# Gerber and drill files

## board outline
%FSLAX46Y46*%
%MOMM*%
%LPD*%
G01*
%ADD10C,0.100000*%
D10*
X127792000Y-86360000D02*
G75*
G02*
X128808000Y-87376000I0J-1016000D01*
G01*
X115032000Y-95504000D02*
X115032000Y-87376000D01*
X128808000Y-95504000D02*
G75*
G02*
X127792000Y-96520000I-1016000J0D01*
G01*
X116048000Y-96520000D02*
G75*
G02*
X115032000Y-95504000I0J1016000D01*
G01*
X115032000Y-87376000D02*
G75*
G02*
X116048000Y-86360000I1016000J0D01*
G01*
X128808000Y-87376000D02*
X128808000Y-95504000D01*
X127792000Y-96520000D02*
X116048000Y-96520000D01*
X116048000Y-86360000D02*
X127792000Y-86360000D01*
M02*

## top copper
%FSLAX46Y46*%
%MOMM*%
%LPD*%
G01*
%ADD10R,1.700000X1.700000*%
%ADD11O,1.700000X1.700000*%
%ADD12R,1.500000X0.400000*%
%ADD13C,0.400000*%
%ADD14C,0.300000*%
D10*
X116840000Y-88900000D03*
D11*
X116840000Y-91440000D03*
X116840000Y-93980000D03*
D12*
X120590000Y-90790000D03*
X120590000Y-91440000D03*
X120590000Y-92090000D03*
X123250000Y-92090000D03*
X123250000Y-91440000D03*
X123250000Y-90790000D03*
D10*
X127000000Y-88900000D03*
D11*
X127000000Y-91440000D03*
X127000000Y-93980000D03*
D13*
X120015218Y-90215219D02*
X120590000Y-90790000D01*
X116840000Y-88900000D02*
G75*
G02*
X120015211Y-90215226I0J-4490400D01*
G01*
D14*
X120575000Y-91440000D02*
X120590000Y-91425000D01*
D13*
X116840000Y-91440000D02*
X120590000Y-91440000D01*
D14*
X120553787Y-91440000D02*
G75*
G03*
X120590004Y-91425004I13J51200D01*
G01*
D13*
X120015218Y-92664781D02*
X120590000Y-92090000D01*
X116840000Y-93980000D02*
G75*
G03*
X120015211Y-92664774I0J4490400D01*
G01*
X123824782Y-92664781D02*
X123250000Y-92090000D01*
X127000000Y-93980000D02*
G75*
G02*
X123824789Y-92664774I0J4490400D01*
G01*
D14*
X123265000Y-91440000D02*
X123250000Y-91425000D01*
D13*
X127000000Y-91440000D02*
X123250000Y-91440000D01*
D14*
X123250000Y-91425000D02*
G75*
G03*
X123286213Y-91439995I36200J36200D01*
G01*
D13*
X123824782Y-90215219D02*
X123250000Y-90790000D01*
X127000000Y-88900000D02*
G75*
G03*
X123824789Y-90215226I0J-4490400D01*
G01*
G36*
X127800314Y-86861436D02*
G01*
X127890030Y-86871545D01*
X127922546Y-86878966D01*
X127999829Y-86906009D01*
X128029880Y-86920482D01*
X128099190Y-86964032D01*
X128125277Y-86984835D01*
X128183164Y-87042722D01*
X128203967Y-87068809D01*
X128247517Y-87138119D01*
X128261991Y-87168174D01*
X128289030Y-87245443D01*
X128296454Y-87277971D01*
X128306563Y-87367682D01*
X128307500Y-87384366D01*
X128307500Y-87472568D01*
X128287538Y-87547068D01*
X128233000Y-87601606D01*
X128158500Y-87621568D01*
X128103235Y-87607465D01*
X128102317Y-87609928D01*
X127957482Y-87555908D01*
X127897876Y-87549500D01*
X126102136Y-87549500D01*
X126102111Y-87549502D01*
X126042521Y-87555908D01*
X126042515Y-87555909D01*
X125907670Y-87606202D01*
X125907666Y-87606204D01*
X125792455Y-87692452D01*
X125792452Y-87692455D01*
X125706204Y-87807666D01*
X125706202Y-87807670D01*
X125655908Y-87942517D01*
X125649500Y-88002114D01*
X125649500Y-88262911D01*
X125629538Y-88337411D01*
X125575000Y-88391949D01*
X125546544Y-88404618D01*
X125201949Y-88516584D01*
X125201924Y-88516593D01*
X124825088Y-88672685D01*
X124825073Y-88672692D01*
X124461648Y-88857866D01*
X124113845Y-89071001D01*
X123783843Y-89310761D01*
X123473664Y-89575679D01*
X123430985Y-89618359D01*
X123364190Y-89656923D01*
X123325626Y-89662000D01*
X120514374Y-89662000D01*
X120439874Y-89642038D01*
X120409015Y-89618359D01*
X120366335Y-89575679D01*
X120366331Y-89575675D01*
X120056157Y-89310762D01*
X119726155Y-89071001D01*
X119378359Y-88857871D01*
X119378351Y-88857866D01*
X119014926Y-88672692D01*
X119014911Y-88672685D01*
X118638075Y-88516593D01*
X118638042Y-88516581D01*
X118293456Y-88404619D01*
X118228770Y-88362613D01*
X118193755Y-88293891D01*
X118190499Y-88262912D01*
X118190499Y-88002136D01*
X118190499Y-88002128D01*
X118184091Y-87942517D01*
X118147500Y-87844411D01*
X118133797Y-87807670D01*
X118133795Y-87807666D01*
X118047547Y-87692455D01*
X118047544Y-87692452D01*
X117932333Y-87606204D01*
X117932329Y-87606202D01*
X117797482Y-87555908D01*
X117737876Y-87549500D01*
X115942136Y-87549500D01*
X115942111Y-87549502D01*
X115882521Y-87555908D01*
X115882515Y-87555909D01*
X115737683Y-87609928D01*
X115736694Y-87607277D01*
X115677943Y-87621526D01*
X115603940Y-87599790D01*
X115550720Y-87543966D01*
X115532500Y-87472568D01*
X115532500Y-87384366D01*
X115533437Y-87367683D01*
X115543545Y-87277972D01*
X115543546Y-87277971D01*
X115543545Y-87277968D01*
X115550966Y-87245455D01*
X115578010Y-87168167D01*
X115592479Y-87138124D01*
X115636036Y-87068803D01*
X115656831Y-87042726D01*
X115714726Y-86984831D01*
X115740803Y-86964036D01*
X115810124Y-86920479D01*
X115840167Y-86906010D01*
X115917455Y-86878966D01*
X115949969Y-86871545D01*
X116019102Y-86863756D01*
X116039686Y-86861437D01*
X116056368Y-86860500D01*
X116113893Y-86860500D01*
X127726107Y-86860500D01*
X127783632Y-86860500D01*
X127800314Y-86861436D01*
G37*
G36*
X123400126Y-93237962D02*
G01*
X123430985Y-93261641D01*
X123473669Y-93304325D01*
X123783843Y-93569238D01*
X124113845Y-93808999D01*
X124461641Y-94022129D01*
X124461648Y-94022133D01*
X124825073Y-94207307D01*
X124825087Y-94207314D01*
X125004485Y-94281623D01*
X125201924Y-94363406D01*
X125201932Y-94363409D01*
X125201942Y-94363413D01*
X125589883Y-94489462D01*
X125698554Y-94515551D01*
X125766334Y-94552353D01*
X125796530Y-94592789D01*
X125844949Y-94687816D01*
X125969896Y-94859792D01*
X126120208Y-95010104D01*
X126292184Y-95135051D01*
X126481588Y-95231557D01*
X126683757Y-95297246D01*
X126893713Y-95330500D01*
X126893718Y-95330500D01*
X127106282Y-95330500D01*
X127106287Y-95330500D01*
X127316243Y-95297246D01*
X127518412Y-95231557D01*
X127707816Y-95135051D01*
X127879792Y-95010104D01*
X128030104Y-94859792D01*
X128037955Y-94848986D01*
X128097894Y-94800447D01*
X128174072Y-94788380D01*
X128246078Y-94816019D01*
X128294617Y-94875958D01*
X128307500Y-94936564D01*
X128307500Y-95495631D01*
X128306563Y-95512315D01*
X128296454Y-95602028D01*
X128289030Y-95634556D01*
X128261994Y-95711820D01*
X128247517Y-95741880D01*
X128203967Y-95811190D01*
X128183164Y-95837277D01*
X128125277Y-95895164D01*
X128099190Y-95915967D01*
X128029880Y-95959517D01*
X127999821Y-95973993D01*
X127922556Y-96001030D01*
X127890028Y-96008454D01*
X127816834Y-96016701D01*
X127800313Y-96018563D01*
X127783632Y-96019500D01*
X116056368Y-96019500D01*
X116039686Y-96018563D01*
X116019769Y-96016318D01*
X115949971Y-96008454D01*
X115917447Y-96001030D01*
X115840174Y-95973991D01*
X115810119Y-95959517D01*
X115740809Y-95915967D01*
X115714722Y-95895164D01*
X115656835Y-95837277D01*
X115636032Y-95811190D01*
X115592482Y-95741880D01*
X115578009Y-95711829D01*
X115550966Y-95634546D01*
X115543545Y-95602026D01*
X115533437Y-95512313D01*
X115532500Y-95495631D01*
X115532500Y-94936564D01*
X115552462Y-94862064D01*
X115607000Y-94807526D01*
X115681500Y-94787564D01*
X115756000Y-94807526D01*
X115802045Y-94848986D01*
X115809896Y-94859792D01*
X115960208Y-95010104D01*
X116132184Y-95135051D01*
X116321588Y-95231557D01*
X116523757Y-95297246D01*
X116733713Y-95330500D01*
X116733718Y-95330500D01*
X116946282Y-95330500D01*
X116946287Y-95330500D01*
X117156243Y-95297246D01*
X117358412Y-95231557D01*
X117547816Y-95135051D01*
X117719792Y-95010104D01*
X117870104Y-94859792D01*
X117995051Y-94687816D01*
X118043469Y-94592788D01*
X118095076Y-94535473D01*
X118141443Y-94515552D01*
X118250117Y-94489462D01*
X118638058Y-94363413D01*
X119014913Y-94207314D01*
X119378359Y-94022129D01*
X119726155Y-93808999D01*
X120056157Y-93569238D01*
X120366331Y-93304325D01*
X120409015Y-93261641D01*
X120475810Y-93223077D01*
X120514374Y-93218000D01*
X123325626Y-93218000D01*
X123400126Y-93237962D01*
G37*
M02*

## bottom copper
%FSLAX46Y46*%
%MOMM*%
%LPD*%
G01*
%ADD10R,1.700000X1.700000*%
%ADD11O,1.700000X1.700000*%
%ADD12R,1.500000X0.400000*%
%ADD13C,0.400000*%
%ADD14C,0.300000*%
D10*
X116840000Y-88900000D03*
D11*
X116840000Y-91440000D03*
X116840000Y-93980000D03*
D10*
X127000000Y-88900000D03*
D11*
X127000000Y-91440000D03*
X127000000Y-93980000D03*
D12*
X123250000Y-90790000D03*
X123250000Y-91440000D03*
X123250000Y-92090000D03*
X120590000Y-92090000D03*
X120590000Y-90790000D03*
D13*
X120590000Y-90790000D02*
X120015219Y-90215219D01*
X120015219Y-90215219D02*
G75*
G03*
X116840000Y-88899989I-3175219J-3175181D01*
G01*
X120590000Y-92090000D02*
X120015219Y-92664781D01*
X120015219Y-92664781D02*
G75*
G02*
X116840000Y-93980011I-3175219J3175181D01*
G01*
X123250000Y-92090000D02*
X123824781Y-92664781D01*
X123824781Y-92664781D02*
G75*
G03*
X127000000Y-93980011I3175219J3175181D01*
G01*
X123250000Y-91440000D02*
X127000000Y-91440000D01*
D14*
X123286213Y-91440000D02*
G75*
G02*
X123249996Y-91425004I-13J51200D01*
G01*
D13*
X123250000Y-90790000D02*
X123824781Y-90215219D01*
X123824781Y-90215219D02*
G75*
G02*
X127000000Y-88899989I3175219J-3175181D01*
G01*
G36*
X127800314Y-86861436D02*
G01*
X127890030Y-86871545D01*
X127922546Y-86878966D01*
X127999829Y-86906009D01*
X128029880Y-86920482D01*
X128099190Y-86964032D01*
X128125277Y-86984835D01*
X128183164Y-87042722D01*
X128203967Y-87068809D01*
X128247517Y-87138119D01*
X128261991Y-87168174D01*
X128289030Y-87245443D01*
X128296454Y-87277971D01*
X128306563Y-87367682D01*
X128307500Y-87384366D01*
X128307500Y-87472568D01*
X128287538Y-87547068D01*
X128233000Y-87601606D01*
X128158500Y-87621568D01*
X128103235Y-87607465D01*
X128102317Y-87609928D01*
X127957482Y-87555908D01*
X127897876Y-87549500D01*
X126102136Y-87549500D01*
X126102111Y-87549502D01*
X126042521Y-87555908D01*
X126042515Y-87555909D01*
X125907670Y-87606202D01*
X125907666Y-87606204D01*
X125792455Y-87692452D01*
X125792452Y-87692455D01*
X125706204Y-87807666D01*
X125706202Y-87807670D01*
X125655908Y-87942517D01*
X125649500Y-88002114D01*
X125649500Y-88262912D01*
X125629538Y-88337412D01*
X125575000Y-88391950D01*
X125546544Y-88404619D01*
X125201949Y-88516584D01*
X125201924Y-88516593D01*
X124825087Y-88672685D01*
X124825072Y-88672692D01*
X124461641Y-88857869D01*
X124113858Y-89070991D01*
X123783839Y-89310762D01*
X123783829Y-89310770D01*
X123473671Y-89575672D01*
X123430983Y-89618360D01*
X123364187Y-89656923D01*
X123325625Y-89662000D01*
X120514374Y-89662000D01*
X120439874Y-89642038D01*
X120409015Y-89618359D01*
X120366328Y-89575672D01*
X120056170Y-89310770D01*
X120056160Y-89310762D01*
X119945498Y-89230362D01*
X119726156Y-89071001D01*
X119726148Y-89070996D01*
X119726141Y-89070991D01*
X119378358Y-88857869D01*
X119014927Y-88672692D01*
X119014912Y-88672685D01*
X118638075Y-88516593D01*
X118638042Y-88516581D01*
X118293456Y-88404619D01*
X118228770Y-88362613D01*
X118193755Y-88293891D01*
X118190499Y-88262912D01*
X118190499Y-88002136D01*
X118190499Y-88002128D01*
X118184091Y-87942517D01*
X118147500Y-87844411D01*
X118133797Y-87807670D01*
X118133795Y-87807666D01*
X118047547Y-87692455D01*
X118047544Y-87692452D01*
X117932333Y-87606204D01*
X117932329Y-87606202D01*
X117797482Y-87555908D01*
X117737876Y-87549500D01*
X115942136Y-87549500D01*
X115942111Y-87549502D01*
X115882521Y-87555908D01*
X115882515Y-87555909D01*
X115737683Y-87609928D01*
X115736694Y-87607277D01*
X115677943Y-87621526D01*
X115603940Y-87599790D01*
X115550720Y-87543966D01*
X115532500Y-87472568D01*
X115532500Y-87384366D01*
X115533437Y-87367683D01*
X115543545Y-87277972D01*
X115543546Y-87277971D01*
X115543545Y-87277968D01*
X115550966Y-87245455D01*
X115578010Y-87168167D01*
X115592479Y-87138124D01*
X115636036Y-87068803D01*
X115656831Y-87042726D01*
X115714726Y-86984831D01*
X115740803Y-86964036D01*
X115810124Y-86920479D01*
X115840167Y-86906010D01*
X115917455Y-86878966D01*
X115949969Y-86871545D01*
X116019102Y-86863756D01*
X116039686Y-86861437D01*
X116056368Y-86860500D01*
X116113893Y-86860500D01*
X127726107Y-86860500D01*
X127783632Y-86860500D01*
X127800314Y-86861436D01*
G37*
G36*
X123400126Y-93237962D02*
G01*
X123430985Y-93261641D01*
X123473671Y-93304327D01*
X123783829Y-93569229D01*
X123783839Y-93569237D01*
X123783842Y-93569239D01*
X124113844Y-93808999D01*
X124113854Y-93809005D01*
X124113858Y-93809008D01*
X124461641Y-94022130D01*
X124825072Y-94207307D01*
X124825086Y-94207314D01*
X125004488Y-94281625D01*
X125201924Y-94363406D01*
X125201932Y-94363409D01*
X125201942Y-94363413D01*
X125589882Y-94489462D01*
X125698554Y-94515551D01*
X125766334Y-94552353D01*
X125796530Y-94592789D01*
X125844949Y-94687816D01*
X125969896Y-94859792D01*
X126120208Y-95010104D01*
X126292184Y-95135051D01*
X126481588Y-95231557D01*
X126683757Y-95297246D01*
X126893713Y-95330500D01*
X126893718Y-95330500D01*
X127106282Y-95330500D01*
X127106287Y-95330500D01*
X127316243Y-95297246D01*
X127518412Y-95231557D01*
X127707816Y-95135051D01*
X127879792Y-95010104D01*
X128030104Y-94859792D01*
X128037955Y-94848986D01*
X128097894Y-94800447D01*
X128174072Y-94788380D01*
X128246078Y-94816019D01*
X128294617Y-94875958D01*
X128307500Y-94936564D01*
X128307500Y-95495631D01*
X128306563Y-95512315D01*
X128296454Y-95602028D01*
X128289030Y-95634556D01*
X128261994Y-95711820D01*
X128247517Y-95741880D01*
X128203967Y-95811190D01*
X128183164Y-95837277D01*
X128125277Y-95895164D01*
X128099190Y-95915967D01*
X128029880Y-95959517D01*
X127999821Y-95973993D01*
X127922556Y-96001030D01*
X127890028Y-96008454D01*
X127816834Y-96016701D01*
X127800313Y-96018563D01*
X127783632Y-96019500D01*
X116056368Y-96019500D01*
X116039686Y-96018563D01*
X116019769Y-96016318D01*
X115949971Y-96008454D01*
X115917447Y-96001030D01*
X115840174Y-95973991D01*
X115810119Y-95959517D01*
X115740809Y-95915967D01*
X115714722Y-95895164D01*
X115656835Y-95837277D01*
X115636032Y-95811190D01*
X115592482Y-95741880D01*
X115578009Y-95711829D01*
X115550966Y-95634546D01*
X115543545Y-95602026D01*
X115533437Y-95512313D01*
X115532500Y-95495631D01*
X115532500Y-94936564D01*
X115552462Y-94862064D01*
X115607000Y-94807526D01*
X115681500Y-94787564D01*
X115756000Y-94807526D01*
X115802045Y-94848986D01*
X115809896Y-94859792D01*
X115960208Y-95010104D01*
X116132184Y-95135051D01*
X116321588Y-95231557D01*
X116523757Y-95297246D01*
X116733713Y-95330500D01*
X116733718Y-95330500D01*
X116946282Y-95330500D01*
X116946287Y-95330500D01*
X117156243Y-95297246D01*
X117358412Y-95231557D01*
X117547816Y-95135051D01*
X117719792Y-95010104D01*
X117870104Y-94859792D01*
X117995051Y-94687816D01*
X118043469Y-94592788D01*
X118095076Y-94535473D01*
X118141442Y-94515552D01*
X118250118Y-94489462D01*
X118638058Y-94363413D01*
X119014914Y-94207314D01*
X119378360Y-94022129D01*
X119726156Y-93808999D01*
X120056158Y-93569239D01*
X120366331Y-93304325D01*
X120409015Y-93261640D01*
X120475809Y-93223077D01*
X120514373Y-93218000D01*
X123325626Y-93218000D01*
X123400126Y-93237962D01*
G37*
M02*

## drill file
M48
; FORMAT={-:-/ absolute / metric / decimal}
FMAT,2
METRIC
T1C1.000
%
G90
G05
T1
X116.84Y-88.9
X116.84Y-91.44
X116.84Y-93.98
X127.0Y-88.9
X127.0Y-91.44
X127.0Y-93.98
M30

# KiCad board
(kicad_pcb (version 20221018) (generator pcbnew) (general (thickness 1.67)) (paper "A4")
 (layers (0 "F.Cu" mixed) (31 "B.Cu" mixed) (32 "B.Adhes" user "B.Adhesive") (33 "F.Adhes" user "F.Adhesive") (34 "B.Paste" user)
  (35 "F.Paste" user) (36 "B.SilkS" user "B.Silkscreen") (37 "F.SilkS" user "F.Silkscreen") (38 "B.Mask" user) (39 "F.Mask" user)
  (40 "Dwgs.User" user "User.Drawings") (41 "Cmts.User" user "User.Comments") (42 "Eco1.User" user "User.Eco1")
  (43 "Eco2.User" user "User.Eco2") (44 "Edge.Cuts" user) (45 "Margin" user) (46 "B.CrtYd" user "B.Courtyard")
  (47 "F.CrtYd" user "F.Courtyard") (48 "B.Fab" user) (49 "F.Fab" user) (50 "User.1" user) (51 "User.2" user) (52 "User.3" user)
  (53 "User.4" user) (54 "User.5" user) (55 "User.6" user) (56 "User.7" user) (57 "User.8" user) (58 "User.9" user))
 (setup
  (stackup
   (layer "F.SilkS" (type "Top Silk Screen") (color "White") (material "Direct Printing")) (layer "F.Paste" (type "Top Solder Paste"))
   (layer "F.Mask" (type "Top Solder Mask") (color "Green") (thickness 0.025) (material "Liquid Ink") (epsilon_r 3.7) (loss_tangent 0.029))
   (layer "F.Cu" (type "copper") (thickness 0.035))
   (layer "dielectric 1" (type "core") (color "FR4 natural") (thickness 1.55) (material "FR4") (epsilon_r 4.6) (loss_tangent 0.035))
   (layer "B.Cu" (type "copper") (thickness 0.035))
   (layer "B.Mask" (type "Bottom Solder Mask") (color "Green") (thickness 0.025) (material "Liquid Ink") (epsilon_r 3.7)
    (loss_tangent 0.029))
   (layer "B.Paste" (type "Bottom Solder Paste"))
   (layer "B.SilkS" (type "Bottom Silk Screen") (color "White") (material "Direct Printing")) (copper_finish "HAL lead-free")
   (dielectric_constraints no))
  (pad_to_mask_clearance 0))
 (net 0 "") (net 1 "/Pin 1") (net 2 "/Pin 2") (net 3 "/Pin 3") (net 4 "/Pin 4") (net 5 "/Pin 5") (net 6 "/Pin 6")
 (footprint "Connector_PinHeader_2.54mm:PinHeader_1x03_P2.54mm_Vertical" (layer "F.Cu") (at 116.84 88.9)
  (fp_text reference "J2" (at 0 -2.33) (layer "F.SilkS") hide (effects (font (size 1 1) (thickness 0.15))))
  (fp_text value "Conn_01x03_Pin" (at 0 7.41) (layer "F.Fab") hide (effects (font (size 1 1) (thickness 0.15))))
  (pad "1" thru_hole rect (at 0 0) (size 1.7 1.7) (drill 1) (layers "*.Cu" "*.Mask") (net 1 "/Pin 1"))
  (pad "2" thru_hole oval (at 0 2.54) (size 1.7 1.7) (drill 1) (layers "*.Cu" "*.Mask") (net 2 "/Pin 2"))
  (pad "3" thru_hole oval (at 0 5.08) (size 1.7 1.7) (drill 1) (layers "*.Cu" "*.Mask") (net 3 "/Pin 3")))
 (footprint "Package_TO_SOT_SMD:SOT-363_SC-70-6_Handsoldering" (layer "F.Cu") (at 121.92 91.44)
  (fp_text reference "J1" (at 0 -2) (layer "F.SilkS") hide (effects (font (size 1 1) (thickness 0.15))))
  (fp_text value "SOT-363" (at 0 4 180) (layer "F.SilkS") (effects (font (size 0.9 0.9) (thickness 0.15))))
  (pad "1" smd rect (at -1.33 -0.65) (size 1.5 0.4) (layers "F.Cu" "F.Paste" "F.Mask") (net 1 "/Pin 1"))
  (pad "2" smd rect (at -1.33 0) (size 1.5 0.4) (layers "F.Cu" "F.Paste" "F.Mask") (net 2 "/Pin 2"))
  (pad "3" smd rect (at -1.33 0.65) (size 1.5 0.4) (layers "F.Cu" "F.Paste" "F.Mask") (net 3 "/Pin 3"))
  (pad "4" smd rect (at 1.33 0.65) (size 1.5 0.4) (layers "F.Cu" "F.Paste" "F.Mask") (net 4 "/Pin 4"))
  (pad "5" smd rect (at 1.33 0) (size 1.5 0.4) (layers "F.Cu" "F.Paste" "F.Mask") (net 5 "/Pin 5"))
  (pad "6" smd rect (at 1.33 -0.65) (size 1.5 0.4) (layers "F.Cu" "F.Paste" "F.Mask") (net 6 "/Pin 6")))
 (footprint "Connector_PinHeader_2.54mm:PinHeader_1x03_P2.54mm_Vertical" (layer "F.Cu") (at 127 88.9)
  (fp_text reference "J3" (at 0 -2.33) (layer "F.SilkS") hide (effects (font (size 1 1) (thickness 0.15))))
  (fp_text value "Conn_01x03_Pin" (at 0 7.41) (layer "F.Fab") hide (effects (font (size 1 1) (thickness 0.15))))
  (pad "1" thru_hole rect (at 0 0) (size 1.7 1.7) (drill 1) (layers "*.Cu" "*.Mask") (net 6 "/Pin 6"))
  (pad "2" thru_hole oval (at 0 2.54) (size 1.7 1.7) (drill 1) (layers "*.Cu" "*.Mask") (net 5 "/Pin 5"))
  (pad "3" thru_hole oval (at 0 5.08) (size 1.7 1.7) (drill 1) (layers "*.Cu" "*.Mask") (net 4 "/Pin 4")))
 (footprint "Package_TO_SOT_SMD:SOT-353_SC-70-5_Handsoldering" (layer "B.Cu") (at 121.92 91.44 180)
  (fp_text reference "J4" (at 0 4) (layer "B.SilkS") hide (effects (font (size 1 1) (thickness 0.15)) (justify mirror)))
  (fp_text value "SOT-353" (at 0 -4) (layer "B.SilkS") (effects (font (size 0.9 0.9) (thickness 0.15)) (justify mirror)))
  (pad "1" smd rect (at -1.33 0.65 180) (size 1.5 0.4) (layers "B.Cu" "B.Paste" "B.Mask") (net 6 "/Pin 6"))
  (pad "2" smd rect (at -1.33 0 180) (size 1.5 0.4) (layers "B.Cu" "B.Paste" "B.Mask") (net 5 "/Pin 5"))
  (pad "3" smd rect (at -1.33 -0.65 180) (size 1.5 0.4) (layers "B.Cu" "B.Paste" "B.Mask") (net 4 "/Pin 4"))
  (pad "4" smd rect (at 1.33 -0.65 180) (size 1.5 0.4) (layers "B.Cu" "B.Paste" "B.Mask") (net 3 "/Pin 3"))
  (pad "5" smd rect (at 1.33 0.65 180) (size 1.5 0.4) (layers "B.Cu" "B.Paste" "B.Mask") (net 1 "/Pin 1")))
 (gr_arc (start 127.792 86.36) (mid 128.51042 86.65758) (end 128.808 87.376) (stroke (width 0.1) (type default)) (layer "Edge.Cuts"))
 (gr_line (start 115.032 95.504) (end 115.032 87.376) (stroke (width 0.1) (type default)) (layer "Edge.Cuts"))
 (gr_arc (start 128.808 95.504) (mid 128.51042 96.22242) (end 127.792 96.52) (stroke (width 0.1) (type default)) (layer "Edge.Cuts"))
 (gr_arc (start 116.048 96.52) (mid 115.32958 96.22242) (end 115.032 95.504) (stroke (width 0.1) (type default)) (layer "Edge.Cuts"))
 (gr_arc (start 115.032 87.376) (mid 115.32958 86.65758) (end 116.048 86.36) (stroke (width 0.1) (type default)) (layer "Edge.Cuts"))
 (gr_line (start 128.808 87.376) (end 128.808 95.504) (stroke (width 0.1) (type default)) (layer "Edge.Cuts"))
 (gr_line (start 127.792 96.52) (end 116.048 96.52) (stroke (width 0.1) (type default)) (layer "Edge.Cuts"))
 (gr_line (start 116.048 86.36) (end 127.792 86.36) (stroke (width 0.1) (type default)) (layer "Edge.Cuts"))
 (segment (start 120.015218 90.215219) (end 120.59 90.79) (width 0.4) (layer "F.Cu") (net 1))
 (arc (start 116.84 88.9) (mid 118.558416 89.241814) (end 120.015218 90.215219) (width 0.4) (layer "F.Cu") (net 1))
 (segment (start 120.59 90.79) (end 120.015219 90.215219) (width 0.4) (layer "B.Cu") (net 1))
 (arc (start 120.015219 90.215219) (mid 118.558416 89.241814) (end 116.84 88.9) (width 0.4) (layer "B.Cu") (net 1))
 (segment (start 120.575 91.44) (end 120.59 91.425) (width 0.3) (layer "F.Cu") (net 2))
 (segment (start 116.84 91.44) (end 120.59 91.44) (width 0.4) (layer "F.Cu") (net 2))
 (arc (start 120.553787 91.44) (mid 120.573385 91.436102) (end 120.59 91.425) (width 0.3) (layer "F.Cu") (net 2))
 (segment (start 120.015218 92.664781) (end 120.59 92.09) (width 0.4) (layer "F.Cu") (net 3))
 (arc (start 116.84 93.98) (mid 118.558416 93.638186) (end 120.015218 92.664781) (width 0.4) (layer "F.Cu") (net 3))
 (segment (start 120.59 92.09) (end 120.015219 92.664781) (width 0.4) (layer "B.Cu") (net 3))
 (arc (start 120.015219 92.664781) (mid 118.558416 93.638186) (end 116.84 93.98) (width 0.4) (layer "B.Cu") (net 3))
 (segment (start 123.824782 92.664781) (end 123.25 92.09) (width 0.4) (layer "F.Cu") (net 4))
 (arc (start 127 93.98) (mid 125.281584 93.638186) (end 123.824782 92.664781) (width 0.4) (layer "F.Cu") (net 4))
 (segment (start 123.25 92.09) (end 123.824781 92.664781) (width 0.4) (layer "B.Cu") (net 4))
 (arc (start 123.824781 92.664781) (mid 125.281584 93.638186) (end 127 93.98) (width 0.4) (layer "B.Cu") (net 4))
 (segment (start 123.265 91.44) (end 123.25 91.425) (width 0.3) (layer "F.Cu") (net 5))
 (segment (start 127 91.44) (end 123.25 91.44) (width 0.4) (layer "F.Cu") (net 5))
 (arc (start 123.25 91.425) (mid 123.266614 91.436102) (end 123.286213 91.44) (width 0.3) (layer "F.Cu") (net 5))
 (segment (start 123.25 91.44) (end 127 91.44) (width 0.4) (layer "B.Cu") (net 5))
 (arc (start 123.286213 91.44) (mid 123.266615 91.436102) (end 123.25 91.425) (width 0.3) (layer "B.Cu") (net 5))
 (segment (start 123.824782 90.215219) (end 123.25 90.79) (width 0.4) (layer "F.Cu") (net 6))
 (arc (start 127 88.9) (mid 125.281584 89.241814) (end 123.824782 90.215219) (width 0.4) (layer "F.Cu") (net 6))
 (segment (start 123.25 90.79) (end 123.824781 90.215219) (width 0.4) (layer "B.Cu") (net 6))
 (arc (start 123.824781 90.215219) (mid 125.281584 89.241814) (end 127 88.9) (width 0.4) (layer "B.Cu") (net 6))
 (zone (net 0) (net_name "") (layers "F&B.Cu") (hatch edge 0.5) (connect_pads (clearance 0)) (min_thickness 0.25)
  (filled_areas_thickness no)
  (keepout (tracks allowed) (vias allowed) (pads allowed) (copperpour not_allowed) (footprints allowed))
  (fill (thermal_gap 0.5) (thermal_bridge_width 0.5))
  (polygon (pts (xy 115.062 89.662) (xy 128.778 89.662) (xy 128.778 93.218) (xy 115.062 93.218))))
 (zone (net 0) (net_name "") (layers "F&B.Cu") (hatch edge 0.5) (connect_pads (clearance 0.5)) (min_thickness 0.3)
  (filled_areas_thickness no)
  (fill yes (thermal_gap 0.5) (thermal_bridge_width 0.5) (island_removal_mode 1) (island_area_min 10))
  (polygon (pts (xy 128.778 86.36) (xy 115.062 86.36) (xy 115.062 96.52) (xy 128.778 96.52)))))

